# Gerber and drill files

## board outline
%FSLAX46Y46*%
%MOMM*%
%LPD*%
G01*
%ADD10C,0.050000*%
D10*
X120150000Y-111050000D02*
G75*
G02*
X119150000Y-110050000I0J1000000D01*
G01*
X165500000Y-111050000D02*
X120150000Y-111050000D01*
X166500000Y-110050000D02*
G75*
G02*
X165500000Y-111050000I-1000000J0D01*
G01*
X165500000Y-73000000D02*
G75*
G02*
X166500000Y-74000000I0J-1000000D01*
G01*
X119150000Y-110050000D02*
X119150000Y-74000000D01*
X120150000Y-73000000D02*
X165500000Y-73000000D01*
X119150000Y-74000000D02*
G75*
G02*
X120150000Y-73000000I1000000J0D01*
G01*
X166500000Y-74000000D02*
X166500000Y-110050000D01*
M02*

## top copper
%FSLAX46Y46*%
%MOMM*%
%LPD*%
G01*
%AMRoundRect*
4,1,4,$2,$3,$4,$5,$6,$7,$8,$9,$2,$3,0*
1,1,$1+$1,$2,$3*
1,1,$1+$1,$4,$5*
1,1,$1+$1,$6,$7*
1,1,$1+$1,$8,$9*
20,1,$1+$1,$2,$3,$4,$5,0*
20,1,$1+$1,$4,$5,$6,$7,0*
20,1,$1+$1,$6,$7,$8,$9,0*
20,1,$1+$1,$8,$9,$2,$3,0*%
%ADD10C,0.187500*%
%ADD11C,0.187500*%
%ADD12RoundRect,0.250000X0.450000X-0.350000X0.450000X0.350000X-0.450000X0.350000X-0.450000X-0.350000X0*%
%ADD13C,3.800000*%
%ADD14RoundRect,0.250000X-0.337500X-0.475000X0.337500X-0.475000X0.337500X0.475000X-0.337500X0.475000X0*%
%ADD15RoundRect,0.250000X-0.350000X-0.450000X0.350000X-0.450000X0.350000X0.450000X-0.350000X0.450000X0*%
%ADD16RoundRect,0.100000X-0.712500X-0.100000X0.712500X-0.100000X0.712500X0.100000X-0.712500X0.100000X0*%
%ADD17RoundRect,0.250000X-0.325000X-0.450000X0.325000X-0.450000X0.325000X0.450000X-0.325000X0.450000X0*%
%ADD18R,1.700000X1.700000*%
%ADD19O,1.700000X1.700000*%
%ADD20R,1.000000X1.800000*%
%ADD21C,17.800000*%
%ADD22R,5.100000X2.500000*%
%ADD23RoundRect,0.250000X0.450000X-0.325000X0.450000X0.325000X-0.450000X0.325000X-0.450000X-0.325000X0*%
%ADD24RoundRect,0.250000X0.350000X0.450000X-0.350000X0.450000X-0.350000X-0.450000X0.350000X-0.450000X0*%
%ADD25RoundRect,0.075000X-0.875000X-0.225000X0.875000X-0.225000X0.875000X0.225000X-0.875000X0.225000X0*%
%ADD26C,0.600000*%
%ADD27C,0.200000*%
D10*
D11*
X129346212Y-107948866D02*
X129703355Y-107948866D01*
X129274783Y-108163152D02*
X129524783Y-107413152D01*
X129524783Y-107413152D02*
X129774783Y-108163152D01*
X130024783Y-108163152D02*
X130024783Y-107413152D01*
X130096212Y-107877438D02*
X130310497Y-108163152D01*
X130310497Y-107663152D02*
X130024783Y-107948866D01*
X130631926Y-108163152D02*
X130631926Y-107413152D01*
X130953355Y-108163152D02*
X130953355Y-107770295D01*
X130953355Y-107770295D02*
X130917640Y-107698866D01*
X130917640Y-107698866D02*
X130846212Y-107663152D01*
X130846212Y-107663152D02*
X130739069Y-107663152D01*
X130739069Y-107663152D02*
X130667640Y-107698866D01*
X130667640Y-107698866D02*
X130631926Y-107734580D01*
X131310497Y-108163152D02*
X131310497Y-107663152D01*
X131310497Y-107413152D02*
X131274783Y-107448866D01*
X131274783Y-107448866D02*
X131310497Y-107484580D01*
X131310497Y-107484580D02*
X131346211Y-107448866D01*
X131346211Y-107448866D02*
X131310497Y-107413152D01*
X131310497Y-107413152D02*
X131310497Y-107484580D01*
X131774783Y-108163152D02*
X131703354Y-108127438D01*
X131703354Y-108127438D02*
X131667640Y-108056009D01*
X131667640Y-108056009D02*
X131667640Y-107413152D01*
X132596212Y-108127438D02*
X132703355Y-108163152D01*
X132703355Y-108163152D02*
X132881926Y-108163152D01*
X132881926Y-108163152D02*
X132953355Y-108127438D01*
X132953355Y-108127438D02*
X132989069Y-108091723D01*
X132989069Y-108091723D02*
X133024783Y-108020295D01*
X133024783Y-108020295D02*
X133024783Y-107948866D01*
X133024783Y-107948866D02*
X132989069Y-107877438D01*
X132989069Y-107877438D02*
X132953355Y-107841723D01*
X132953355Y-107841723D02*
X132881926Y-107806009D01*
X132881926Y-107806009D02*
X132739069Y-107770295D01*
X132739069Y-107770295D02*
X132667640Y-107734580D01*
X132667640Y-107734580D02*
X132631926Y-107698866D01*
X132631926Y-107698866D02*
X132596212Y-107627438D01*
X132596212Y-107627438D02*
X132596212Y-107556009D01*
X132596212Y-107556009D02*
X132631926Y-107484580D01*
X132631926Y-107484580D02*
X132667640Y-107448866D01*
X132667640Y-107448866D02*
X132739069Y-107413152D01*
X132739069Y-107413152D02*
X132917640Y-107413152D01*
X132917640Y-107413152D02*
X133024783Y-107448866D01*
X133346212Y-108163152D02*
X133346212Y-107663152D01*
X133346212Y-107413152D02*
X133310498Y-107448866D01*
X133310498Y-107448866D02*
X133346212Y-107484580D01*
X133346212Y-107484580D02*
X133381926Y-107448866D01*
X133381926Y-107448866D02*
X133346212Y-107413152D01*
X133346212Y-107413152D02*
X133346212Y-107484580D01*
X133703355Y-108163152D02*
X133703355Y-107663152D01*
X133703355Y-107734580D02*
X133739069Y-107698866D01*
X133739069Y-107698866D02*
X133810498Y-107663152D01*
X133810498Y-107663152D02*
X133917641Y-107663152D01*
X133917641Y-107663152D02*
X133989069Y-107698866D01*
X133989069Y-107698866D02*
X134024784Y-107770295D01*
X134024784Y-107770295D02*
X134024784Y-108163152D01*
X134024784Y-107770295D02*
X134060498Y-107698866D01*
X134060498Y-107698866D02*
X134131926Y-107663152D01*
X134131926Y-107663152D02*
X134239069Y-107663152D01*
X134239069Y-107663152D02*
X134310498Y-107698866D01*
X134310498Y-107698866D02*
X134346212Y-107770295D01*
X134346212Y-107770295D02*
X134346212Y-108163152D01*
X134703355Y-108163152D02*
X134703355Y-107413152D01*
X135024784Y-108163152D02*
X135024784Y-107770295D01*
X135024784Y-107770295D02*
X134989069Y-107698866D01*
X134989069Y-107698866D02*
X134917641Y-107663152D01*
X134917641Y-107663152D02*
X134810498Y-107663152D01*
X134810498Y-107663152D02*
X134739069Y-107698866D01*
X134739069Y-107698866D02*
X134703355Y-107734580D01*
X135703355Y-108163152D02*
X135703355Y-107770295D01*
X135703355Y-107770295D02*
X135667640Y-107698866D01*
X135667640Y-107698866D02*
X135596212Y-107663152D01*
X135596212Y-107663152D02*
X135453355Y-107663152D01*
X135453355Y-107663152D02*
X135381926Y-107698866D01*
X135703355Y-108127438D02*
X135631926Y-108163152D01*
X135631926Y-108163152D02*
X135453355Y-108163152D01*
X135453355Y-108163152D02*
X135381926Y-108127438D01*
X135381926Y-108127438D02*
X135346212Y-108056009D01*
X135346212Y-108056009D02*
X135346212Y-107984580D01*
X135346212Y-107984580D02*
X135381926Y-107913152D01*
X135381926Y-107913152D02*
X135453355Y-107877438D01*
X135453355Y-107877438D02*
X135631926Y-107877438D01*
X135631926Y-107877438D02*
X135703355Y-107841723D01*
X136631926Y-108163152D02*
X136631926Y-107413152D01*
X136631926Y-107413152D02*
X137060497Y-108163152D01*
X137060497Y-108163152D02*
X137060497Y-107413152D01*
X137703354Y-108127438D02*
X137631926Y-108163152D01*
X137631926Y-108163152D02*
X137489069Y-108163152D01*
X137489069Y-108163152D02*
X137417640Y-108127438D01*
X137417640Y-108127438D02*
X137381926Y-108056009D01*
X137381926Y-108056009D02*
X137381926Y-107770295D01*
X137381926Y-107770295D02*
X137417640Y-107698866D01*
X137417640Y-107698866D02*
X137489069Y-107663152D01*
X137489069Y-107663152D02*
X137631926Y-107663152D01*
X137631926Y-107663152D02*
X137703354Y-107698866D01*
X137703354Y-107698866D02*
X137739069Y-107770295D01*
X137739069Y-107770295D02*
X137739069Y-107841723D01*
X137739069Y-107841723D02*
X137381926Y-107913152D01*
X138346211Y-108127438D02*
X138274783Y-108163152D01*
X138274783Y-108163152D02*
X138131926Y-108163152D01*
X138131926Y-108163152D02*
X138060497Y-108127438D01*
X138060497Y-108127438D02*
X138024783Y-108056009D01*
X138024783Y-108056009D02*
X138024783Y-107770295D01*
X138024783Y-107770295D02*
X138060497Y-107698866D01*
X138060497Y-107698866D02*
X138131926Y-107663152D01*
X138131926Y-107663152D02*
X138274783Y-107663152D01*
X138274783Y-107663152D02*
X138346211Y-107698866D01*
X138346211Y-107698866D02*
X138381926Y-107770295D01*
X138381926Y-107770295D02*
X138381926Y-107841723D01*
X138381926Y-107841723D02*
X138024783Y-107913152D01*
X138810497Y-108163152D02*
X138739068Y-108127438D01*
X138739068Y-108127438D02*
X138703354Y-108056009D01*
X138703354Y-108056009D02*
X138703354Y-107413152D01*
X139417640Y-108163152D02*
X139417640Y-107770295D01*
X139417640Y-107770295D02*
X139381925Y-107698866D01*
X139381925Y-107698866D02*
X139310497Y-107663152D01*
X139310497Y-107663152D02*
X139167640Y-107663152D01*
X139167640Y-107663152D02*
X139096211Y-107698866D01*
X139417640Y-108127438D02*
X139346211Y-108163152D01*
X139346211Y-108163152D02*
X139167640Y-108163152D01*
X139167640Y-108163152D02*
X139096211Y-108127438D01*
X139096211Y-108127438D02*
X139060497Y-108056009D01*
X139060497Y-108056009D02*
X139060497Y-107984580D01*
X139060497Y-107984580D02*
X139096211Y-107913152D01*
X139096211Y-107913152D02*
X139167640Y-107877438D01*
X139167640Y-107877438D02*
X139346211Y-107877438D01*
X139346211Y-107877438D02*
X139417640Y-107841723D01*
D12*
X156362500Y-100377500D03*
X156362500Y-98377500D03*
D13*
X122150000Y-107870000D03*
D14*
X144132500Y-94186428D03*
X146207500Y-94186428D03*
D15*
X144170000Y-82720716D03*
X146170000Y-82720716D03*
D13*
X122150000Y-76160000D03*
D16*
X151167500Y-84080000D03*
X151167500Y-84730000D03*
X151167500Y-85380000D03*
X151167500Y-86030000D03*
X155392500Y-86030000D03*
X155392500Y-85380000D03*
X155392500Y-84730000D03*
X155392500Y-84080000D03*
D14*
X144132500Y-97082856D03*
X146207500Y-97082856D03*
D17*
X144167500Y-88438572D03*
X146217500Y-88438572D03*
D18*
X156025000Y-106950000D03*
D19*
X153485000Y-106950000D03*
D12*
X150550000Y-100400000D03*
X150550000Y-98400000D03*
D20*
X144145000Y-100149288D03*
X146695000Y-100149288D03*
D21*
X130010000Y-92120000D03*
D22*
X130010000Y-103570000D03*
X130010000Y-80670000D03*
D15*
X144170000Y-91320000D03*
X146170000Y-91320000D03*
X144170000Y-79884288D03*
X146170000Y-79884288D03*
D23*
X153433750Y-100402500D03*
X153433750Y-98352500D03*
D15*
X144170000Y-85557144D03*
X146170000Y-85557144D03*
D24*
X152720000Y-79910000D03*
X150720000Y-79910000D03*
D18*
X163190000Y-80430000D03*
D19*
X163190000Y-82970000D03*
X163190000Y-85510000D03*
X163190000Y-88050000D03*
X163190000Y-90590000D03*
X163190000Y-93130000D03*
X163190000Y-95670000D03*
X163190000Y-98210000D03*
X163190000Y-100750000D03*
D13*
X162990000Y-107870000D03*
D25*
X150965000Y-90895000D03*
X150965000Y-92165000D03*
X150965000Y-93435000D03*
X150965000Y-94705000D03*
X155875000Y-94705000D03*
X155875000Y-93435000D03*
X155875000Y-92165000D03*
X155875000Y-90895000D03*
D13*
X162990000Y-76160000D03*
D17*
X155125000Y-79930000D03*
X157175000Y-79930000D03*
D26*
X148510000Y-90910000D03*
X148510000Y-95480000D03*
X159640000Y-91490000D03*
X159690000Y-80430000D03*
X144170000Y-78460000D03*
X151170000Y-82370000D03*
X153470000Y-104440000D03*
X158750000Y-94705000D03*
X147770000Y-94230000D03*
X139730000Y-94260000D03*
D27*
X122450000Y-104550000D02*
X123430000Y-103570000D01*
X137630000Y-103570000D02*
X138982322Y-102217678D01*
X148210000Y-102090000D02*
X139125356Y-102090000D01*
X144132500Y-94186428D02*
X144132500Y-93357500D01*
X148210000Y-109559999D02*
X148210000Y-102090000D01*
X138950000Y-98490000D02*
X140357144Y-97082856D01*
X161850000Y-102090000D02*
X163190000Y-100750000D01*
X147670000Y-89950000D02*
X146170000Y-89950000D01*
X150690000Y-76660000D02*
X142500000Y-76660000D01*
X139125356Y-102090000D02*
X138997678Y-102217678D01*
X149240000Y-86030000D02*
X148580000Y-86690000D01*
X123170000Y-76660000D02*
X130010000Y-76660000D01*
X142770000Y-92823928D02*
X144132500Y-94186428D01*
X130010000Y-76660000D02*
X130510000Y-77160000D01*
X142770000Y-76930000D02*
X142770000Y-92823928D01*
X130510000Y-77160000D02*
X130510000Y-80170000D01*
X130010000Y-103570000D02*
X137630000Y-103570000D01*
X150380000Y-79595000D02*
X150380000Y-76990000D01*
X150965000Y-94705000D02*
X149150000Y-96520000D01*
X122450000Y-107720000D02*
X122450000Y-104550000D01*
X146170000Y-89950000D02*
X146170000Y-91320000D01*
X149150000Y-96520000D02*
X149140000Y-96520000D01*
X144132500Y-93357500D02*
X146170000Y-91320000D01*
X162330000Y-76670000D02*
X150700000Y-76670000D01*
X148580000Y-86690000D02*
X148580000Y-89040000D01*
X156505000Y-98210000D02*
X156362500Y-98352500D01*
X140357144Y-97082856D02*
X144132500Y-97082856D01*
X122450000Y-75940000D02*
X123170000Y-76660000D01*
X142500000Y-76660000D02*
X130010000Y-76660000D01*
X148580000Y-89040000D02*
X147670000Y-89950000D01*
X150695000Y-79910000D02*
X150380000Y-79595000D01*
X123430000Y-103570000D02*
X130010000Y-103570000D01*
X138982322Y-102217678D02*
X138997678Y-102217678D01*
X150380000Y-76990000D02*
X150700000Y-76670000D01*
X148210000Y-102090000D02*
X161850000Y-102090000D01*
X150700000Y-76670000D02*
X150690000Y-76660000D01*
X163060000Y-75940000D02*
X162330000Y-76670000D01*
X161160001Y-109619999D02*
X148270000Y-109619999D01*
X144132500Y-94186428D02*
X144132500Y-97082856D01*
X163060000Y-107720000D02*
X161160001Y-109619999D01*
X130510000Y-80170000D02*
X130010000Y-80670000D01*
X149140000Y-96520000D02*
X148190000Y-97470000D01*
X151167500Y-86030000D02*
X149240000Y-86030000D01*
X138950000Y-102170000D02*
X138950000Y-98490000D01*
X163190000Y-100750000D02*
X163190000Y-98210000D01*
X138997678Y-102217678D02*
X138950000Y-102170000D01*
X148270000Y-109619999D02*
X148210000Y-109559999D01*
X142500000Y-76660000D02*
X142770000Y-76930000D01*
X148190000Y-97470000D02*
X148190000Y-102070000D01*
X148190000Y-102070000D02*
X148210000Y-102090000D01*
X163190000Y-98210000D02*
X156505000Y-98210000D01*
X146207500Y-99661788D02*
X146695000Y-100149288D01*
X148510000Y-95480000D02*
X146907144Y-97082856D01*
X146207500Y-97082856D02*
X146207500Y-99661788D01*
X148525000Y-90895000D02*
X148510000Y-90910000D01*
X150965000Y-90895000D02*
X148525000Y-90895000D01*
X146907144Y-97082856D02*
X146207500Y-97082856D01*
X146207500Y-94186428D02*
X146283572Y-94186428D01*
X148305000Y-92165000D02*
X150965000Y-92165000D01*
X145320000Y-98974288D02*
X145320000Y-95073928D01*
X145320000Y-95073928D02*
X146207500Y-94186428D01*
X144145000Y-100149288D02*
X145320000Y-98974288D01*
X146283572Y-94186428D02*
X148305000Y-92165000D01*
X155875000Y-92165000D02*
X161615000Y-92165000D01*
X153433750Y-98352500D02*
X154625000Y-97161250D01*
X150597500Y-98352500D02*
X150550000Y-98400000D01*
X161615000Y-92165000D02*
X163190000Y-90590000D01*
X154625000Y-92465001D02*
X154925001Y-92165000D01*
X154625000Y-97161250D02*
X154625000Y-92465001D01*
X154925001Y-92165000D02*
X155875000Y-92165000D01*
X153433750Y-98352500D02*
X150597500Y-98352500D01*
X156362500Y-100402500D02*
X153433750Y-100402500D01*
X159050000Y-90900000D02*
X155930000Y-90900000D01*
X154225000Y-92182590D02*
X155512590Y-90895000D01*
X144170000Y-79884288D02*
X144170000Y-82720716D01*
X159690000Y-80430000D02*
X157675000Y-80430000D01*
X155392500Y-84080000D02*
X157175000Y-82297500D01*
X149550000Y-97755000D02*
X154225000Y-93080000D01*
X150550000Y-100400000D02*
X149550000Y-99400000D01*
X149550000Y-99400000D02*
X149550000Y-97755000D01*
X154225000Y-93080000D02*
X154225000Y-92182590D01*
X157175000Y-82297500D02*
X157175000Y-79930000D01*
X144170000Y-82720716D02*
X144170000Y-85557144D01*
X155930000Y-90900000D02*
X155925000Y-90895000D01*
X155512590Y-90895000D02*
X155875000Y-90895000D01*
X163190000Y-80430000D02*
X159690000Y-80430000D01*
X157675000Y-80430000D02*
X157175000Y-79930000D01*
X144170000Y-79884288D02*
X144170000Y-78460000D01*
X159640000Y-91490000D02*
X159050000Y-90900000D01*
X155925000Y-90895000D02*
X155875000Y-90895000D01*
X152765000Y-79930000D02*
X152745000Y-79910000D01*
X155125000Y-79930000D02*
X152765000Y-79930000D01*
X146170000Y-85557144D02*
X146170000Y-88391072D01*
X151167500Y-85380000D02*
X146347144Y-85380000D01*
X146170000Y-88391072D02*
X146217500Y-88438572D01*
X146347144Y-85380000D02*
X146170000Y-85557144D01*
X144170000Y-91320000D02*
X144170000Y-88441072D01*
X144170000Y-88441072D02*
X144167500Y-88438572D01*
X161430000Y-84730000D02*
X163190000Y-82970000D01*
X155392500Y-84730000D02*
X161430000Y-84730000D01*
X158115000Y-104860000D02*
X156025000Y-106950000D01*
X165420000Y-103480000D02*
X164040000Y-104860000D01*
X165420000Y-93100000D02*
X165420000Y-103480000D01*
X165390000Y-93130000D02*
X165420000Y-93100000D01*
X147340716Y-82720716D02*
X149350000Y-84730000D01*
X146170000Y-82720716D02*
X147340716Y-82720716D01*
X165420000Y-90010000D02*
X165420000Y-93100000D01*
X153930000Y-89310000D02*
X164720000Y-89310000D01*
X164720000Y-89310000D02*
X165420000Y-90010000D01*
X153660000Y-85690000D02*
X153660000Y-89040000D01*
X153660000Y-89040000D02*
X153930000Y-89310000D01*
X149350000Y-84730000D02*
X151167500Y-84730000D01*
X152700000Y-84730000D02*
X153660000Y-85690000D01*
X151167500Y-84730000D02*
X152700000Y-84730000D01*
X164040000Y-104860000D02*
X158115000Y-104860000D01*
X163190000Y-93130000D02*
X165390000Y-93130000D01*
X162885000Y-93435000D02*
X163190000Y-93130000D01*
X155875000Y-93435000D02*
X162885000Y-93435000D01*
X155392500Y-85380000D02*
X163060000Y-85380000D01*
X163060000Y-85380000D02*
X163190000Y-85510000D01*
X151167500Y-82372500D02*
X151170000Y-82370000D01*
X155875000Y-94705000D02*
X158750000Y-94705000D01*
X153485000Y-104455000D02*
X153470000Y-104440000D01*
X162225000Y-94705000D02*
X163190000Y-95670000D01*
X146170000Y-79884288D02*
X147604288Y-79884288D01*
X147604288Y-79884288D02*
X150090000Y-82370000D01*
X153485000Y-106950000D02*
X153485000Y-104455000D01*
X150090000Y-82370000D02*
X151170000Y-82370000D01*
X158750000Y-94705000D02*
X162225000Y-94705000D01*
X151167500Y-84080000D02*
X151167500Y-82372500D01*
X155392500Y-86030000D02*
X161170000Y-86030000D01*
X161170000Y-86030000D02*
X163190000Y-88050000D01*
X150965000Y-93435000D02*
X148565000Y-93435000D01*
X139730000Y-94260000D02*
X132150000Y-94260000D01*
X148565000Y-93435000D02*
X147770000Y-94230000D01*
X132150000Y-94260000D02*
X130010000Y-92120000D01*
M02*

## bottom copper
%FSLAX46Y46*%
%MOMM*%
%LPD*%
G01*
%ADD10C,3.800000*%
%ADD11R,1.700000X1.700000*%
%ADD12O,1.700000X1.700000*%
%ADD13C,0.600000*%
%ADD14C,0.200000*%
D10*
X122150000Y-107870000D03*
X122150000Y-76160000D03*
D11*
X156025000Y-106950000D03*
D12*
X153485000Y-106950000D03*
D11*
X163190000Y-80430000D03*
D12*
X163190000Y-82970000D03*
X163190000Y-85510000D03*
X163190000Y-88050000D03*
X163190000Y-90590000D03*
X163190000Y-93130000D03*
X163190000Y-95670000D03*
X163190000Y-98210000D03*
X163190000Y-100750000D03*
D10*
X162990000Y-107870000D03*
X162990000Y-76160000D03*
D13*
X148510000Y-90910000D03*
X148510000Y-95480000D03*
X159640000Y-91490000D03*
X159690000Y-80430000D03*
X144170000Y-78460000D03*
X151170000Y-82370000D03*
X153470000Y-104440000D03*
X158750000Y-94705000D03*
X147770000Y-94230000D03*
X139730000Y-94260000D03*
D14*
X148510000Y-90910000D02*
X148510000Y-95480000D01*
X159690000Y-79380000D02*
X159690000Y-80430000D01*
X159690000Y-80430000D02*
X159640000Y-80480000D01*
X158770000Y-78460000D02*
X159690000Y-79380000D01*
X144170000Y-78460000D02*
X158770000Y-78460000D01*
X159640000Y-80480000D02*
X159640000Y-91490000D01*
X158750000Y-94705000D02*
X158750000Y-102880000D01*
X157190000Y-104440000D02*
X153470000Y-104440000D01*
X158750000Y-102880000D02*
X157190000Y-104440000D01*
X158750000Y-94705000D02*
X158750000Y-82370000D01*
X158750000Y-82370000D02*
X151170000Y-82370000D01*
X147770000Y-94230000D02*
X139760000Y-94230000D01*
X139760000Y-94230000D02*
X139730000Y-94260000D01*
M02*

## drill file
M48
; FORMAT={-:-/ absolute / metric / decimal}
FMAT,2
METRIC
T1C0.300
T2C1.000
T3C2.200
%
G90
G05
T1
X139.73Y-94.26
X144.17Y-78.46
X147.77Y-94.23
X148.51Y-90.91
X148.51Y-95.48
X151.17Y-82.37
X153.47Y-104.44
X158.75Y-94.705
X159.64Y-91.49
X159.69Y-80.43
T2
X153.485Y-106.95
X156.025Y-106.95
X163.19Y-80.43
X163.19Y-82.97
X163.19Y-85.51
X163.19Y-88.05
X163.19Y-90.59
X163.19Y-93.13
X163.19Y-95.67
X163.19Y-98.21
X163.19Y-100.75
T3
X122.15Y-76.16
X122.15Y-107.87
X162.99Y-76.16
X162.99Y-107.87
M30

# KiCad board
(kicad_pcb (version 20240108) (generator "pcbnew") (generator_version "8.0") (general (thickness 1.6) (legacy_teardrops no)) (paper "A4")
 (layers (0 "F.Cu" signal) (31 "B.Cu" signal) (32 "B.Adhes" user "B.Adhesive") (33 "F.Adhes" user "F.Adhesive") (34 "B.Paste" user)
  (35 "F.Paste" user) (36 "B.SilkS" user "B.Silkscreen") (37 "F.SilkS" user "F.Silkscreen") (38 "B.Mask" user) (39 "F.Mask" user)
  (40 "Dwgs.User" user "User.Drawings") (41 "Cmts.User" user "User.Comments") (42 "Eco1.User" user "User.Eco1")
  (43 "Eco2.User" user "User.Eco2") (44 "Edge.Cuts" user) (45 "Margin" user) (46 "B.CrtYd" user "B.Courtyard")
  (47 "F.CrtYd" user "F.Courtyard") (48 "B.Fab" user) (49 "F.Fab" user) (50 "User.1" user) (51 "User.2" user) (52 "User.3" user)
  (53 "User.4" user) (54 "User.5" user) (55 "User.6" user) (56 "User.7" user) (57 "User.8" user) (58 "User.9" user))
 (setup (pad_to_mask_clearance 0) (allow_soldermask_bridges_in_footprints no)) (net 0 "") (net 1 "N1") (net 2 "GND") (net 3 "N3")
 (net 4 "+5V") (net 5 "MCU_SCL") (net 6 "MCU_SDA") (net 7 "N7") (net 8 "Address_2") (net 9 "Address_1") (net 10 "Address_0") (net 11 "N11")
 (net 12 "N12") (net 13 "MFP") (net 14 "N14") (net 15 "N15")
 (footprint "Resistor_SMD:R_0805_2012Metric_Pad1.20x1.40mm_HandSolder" (layer "F.Cu") (at 156.3625 99.3775 90)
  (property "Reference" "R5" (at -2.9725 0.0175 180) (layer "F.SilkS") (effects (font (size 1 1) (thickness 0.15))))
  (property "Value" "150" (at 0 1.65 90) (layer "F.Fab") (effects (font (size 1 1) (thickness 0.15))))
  (pad "1" smd roundrect (at -1 0 90) (size 1.2 1.4) (layers "F.Cu" "F.Paste" "F.Mask") (roundrect_rratio 0.208333) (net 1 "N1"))
  (pad "2" smd roundrect (at 1 0 90) (size 1.2 1.4) (layers "F.Cu" "F.Paste" "F.Mask") (roundrect_rratio 0.208333) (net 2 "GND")))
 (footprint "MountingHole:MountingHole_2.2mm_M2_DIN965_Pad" (layer "F.Cu") (at 122.15 107.87)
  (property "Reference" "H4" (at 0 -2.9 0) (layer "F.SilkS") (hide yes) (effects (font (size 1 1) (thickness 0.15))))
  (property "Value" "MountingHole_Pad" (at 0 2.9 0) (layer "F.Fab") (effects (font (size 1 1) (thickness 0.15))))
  (pad "1" thru_hole circle (at 0 0) (size 3.8 3.8) (drill 2.2) (layers "*.Cu" "*.Mask") (remove_unused_layers no) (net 2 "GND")))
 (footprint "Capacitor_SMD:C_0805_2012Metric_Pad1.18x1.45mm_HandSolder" (layer "F.Cu") (at 145.17 94.186428)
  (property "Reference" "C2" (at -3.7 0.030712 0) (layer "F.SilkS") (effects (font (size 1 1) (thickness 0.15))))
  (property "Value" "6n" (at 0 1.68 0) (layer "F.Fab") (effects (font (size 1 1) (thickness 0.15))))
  (pad "1" smd roundrect (at -1.0375 0) (size 1.175 1.45) (layers "F.Cu" "F.Paste" "F.Mask") (roundrect_rratio 0.212766) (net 2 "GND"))
  (pad "2" smd roundrect (at 1.0375 0) (size 1.175 1.45) (layers "F.Cu" "F.Paste" "F.Mask") (roundrect_rratio 0.212766) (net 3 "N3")))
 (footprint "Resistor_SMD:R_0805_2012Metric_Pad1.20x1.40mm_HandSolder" (layer "F.Cu") (at 145.17 82.720716)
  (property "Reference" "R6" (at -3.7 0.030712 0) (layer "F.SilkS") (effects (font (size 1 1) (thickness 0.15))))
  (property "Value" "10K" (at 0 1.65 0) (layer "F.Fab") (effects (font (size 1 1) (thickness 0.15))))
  (pad "1" smd roundrect (at -1 0) (size 1.2 1.4) (layers "F.Cu" "F.Paste" "F.Mask") (roundrect_rratio 0.208333) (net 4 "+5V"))
  (pad "2" smd roundrect (at 1 0) (size 1.2 1.4) (layers "F.Cu" "F.Paste" "F.Mask") (roundrect_rratio 0.208333) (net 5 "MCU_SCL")))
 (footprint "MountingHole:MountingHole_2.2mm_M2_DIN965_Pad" (layer "F.Cu") (at 122.15 76.16)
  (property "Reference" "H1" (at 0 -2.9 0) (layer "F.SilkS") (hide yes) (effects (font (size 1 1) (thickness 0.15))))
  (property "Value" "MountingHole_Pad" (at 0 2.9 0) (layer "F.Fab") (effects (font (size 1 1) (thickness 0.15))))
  (pad "1" thru_hole circle (at 0 0) (size 3.8 3.8) (drill 2.2) (layers "*.Cu" "*.Mask") (remove_unused_layers no) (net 2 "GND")))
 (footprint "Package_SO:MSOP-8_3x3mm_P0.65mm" (layer "F.Cu") (at 153.28 85.055)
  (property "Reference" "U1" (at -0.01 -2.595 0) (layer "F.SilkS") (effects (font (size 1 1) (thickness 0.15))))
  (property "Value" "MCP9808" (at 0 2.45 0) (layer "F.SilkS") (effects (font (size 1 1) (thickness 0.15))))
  (pad "1" smd roundrect (at -2.1125 -0.975) (size 1.625 0.4) (layers "F.Cu" "F.Paste" "F.Mask") (roundrect_rratio 0.25) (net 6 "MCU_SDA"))
  (pad "2" smd roundrect (at -2.1125 -0.325) (size 1.625 0.4) (layers "F.Cu" "F.Paste" "F.Mask") (roundrect_rratio 0.25) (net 5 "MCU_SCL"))
  (pad "3" smd roundrect (at -2.1125 0.325) (size 1.625 0.4) (layers "F.Cu" "F.Paste" "F.Mask") (roundrect_rratio 0.25) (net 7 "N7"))
  (pad "4" smd roundrect (at -2.1125 0.975) (size 1.625 0.4) (layers "F.Cu" "F.Paste" "F.Mask") (roundrect_rratio 0.25) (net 2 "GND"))
  (pad "5" smd roundrect (at 2.1125 0.975) (size 1.625 0.4) (layers "F.Cu" "F.Paste" "F.Mask") (roundrect_rratio 0.25) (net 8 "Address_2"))
  (pad "6" smd roundrect (at 2.1125 0.325) (size 1.625 0.4) (layers "F.Cu" "F.Paste" "F.Mask") (roundrect_rratio 0.25) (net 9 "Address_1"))
  (pad "7" smd roundrect (at 2.1125 -0.325) (size 1.625 0.4) (layers "F.Cu" "F.Paste" "F.Mask") (roundrect_rratio 0.25) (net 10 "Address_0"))
  (pad "8" smd roundrect (at 2.1125 -0.975) (size 1.625 0.4) (layers "F.Cu" "F.Paste" "F.Mask") (roundrect_rratio 0.25) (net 4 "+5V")))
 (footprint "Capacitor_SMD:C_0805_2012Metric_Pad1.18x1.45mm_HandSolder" (layer "F.Cu") (at 145.17 97.082856)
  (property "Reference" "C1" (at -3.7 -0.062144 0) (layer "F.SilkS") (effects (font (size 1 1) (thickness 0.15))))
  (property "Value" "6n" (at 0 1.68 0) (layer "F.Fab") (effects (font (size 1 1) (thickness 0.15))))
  (pad "1" smd roundrect (at -1.0375 0) (size 1.175 1.45) (layers "F.Cu" "F.Paste" "F.Mask") (roundrect_rratio 0.212766) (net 2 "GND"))
  (pad "2" smd roundrect (at 1.0375 0) (size 1.175 1.45) (layers "F.Cu" "F.Paste" "F.Mask") (roundrect_rratio 0.212766) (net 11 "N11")))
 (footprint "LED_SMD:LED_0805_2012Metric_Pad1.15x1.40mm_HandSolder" (layer "F.Cu") (at 145.1925 88.438572)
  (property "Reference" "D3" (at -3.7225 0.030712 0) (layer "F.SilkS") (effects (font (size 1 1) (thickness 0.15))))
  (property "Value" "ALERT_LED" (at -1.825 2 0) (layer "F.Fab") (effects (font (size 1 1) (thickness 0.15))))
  (pad "1" smd roundrect (at -1.025 0) (size 1.15 1.4) (layers "F.Cu" "F.Paste" "F.Mask") (roundrect_rratio 0.217391) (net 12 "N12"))
  (pad "2" smd roundrect (at 1.025 0) (size 1.15 1.4) (layers "F.Cu" "F.Paste" "F.Mask") (roundrect_rratio 0.217391) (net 7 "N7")))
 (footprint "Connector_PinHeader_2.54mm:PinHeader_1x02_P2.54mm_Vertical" (layer "F.Cu") (at 156.025 106.95 -90)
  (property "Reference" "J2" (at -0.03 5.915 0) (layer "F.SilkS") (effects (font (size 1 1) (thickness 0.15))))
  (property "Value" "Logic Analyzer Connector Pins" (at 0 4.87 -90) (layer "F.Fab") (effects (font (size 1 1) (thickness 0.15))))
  (pad "1" thru_hole rect (at 0 0 270) (size 1.7 1.7) (drill 1) (layers "*.Cu" "*.Mask") (remove_unused_layers no) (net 5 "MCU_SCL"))
  (pad "2" thru_hole oval (at 0 2.54 270) (size 1.7 1.7) (drill 1) (layers "*.Cu" "*.Mask") (remove_unused_layers no) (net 6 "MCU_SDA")))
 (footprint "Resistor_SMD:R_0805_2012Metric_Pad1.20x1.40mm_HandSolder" (layer "F.Cu") (at 150.55 99.4 90)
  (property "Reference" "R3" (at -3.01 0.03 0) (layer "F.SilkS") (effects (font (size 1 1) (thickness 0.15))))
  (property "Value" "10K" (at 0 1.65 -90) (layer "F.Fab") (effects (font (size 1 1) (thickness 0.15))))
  (pad "1" smd roundrect (at -1 0 90) (size 1.2 1.4) (layers "F.Cu" "F.Paste" "F.Mask") (roundrect_rratio 0.208333) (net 4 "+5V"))
  (pad "2" smd roundrect (at 1 0 90) (size 1.2 1.4) (layers "F.Cu" "F.Paste" "F.Mask") (roundrect_rratio 0.208333) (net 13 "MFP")))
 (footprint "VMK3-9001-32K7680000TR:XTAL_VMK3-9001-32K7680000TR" (layer "F.Cu") (at 145.42 100.149288)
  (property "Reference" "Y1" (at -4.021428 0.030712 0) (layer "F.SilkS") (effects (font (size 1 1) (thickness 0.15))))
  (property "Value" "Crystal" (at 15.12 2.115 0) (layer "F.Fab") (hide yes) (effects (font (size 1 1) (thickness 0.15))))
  (pad "1" smd rect (at -1.275 0) (size 1 1.8) (layers "F.Cu" "F.Paste" "F.Mask") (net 3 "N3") (solder_mask_margin 0.102))
  (pad "2" smd rect (at 1.275 0) (size 1 1.8) (layers "F.Cu" "F.Paste" "F.Mask") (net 11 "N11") (solder_mask_margin 0.102)))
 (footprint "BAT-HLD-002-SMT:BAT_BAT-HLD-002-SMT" (layer "F.Cu") (at 130.01 92.12 90)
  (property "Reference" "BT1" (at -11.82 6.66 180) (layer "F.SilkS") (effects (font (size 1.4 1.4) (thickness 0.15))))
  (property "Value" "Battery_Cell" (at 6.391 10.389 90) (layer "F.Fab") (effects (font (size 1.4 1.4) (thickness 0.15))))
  (pad "N" smd circle (at 0 0 90) (size 17.8 17.8) (layers "F.Cu" "F.Mask") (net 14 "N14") (solder_mask_margin 0.102))
  (pad "P1" smd rect (at -11.45 0 90) (size 2.5 5.1) (layers "F.Cu" "F.Paste" "F.Mask") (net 2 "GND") (solder_mask_margin 0.102))
  (pad "P2" smd rect (at 11.45 0 90) (size 2.5 5.1) (layers "F.Cu" "F.Paste" "F.Mask") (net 2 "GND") (solder_mask_margin 0.102)))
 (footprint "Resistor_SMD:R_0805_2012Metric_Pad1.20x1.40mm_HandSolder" (layer "F.Cu") (at 145.17 91.32)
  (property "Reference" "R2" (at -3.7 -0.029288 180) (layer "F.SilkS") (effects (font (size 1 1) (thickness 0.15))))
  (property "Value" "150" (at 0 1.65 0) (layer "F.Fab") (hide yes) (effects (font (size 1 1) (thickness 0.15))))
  (pad "1" smd roundrect (at -1 0) (size 1.2 1.4) (layers "F.Cu" "F.Paste" "F.Mask") (roundrect_rratio 0.208333) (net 12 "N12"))
  (pad "2" smd roundrect (at 1 0) (size 1.2 1.4) (layers "F.Cu" "F.Paste" "F.Mask") (roundrect_rratio 0.208333) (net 2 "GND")))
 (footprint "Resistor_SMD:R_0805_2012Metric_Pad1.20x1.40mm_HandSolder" (layer "F.Cu") (at 145.17 79.884288)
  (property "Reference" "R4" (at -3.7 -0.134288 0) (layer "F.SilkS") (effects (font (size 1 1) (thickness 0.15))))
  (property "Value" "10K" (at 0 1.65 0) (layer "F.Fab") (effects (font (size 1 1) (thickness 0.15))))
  (pad "1" smd roundrect (at -1 0) (size 1.2 1.4) (layers "F.Cu" "F.Paste" "F.Mask") (roundrect_rratio 0.208333) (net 4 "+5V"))
  (pad "2" smd roundrect (at 1 0) (size 1.2 1.4) (layers "F.Cu" "F.Paste" "F.Mask") (roundrect_rratio 0.208333) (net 6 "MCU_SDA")))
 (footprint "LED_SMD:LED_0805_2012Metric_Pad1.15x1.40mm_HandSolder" (layer "F.Cu") (at 153.43375 99.3775 90)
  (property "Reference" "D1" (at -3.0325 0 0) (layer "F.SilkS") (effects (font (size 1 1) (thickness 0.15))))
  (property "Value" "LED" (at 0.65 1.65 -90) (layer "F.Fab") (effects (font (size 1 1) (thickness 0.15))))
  (pad "1" smd roundrect (at -1.025 0 90) (size 1.15 1.4) (layers "F.Cu" "F.Paste" "F.Mask") (roundrect_rratio 0.217391) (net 1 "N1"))
  (pad "2" smd roundrect (at 1.025 0 90) (size 1.15 1.4) (layers "F.Cu" "F.Paste" "F.Mask") (roundrect_rratio 0.217391) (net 13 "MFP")))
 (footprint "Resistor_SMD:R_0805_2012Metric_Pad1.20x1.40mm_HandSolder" (layer "F.Cu") (at 145.17 85.557144)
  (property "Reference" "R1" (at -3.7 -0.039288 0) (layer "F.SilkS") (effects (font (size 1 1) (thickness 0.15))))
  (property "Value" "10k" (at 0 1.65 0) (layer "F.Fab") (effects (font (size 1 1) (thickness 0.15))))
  (pad "1" smd roundrect (at -1 0) (size 1.2 1.4) (layers "F.Cu" "F.Paste" "F.Mask") (roundrect_rratio 0.208333) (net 4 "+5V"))
  (pad "2" smd roundrect (at 1 0) (size 1.2 1.4) (layers "F.Cu" "F.Paste" "F.Mask") (roundrect_rratio 0.208333) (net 7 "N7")))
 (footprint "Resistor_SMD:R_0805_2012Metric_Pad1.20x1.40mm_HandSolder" (layer "F.Cu") (at 151.72 79.91 180)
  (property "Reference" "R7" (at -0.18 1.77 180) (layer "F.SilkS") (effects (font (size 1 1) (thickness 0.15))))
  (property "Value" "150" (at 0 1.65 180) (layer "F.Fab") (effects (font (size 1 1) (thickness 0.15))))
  (pad "1" smd roundrect (at -1 0 180) (size 1.2 1.4) (layers "F.Cu" "F.Paste" "F.Mask") (roundrect_rratio 0.208333) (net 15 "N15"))
  (pad "2" smd roundrect (at 1 0 180) (size 1.2 1.4) (layers "F.Cu" "F.Paste" "F.Mask") (roundrect_rratio 0.208333) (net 2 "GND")))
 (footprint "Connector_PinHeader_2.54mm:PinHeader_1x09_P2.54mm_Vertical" (layer "F.Cu") (at 163.19 80.43)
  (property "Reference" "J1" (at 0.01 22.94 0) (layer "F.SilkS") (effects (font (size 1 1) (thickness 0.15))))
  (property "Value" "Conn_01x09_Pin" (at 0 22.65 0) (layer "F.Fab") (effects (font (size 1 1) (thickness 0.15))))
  (pad "1" thru_hole rect (at 0 0) (size 1.7 1.7) (drill 1) (layers "*.Cu" "*.Mask") (remove_unused_layers no) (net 4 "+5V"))
  (pad "2" thru_hole oval (at 0 2.54) (size 1.7 1.7) (drill 1) (layers "*.Cu" "*.Mask") (remove_unused_layers no) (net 10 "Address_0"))
  (pad "3" thru_hole oval (at 0 5.08) (size 1.7 1.7) (drill 1) (layers "*.Cu" "*.Mask") (remove_unused_layers no) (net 9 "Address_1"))
  (pad "4" thru_hole oval (at 0 7.62) (size 1.7 1.7) (drill 1) (layers "*.Cu" "*.Mask") (remove_unused_layers no) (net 8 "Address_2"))
  (pad "5" thru_hole oval (at 0 10.16) (size 1.7 1.7) (drill 1) (layers "*.Cu" "*.Mask") (remove_unused_layers no) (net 13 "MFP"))
  (pad "6" thru_hole oval (at 0 12.7) (size 1.7 1.7) (drill 1) (layers "*.Cu" "*.Mask") (remove_unused_layers no) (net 5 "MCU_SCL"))
  (pad "7" thru_hole oval (at 0 15.24) (size 1.7 1.7) (drill 1) (layers "*.Cu" "*.Mask") (remove_unused_layers no) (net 6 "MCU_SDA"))
  (pad "8" thru_hole oval (at 0 17.78) (size 1.7 1.7) (drill 1) (layers "*.Cu" "*.Mask") (remove_unused_layers no) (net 2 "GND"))
  (pad "9" thru_hole oval (at 0 20.32) (size 1.7 1.7) (drill 1) (layers "*.Cu" "*.Mask") (remove_unused_layers no) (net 2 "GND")))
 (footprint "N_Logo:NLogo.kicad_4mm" (layer "F.Cu") (at 127.06 107.719644)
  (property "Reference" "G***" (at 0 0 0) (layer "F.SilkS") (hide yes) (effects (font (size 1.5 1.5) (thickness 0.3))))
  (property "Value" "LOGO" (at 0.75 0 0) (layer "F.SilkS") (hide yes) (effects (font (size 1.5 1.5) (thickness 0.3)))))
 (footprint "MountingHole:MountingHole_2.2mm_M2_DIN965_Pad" (layer "F.Cu") (at 162.99 107.87)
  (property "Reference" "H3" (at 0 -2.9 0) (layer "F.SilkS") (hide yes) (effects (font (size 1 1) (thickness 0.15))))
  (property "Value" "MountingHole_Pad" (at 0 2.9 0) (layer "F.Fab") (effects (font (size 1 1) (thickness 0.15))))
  (pad "1" thru_hole circle (at 0 0) (size 3.8 3.8) (drill 2.2) (layers "*.Cu" "*.Mask") (remove_unused_layers no) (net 2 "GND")))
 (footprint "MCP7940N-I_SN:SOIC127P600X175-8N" (layer "F.Cu") (at 153.42 92.8)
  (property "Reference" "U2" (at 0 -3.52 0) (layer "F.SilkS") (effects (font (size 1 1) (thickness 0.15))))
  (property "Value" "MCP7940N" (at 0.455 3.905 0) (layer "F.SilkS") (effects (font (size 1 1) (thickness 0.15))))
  (pad "1" smd roundrect (at -2.455 -1.905) (size 1.9 0.6) (layers "F.Cu" "F.Paste" "F.Mask") (roundrect_rratio 0.125) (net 11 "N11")
   (solder_mask_margin 0.102))
  (pad "2" smd roundrect (at -2.455 -0.635) (size 1.9 0.6) (layers "F.Cu" "F.Paste" "F.Mask") (roundrect_rratio 0.125) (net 3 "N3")
   (solder_mask_margin 0.102))
  (pad "3" smd roundrect (at -2.455 0.635) (size 1.9 0.6) (layers "F.Cu" "F.Paste" "F.Mask") (roundrect_rratio 0.125) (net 14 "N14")
   (solder_mask_margin 0.102))
  (pad "4" smd roundrect (at -2.455 1.905) (size 1.9 0.6) (layers "F.Cu" "F.Paste" "F.Mask") (roundrect_rratio 0.125) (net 2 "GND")
   (solder_mask_margin 0.102))
  (pad "5" smd roundrect (at 2.455 1.905) (size 1.9 0.6) (layers "F.Cu" "F.Paste" "F.Mask") (roundrect_rratio 0.125) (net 6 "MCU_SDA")
   (solder_mask_margin 0.102))
  (pad "6" smd roundrect (at 2.455 0.635) (size 1.9 0.6) (layers "F.Cu" "F.Paste" "F.Mask") (roundrect_rratio 0.125) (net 5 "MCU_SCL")
   (solder_mask_margin 0.102))
  (pad "7" smd roundrect (at 2.455 -0.635) (size 1.9 0.6) (layers "F.Cu" "F.Paste" "F.Mask") (roundrect_rratio 0.125) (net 13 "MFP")
   (solder_mask_margin 0.102))
  (pad "8" smd roundrect (at 2.455 -1.905) (size 1.9 0.6) (layers "F.Cu" "F.Paste" "F.Mask") (roundrect_rratio 0.125) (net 4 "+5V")
   (solder_mask_margin 0.102)))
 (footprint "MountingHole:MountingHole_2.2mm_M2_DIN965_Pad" (layer "F.Cu") (at 162.99 76.16)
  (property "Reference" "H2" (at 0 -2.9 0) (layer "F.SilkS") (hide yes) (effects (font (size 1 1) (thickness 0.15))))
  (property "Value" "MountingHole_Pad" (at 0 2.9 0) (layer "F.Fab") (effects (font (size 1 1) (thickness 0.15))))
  (pad "1" thru_hole circle (at 0 0) (size 3.8 3.8) (drill 2.2) (layers "*.Cu" "*.Mask") (remove_unused_layers no) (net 2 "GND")))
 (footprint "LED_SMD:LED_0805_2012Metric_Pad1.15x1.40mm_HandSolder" (layer "F.Cu") (at 156.15 79.93)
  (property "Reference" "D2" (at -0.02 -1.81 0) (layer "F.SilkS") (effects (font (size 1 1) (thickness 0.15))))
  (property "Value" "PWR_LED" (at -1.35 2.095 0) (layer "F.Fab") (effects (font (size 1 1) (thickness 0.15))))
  (pad "1" smd roundrect (at -1.025 0) (size 1.15 1.4) (layers "F.Cu" "F.Paste" "F.Mask") (roundrect_rratio 0.217391) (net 15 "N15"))
  (pad "2" smd roundrect (at 1.025 0) (size 1.15 1.4) (layers "F.Cu" "F.Paste" "F.Mask") (roundrect_rratio 0.217391) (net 4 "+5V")))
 (gr_arc (start 120.15 111.05) (mid 119.442893 110.757107) (end 119.15 110.05) (stroke (width 0.05) (type default)) (layer "Edge.Cuts"))
 (gr_line (start 165.5 111.05) (end 120.15 111.05) (stroke (width 0.05) (type default)) (layer "Edge.Cuts"))
 (gr_arc (start 166.5 110.05) (mid 166.207107 110.757107) (end 165.5 111.05) (stroke (width 0.05) (type default)) (layer "Edge.Cuts"))
 (gr_arc (start 165.5 73) (mid 166.207107 73.292893) (end 166.5 74) (stroke (width 0.05) (type default)) (layer "Edge.Cuts"))
 (gr_line (start 119.15 110.05) (end 119.15 74) (stroke (width 0.05) (type default)) (layer "Edge.Cuts"))
 (gr_line (start 120.15 73) (end 165.5 73) (stroke (width 0.05) (type default)) (layer "Edge.Cuts"))
 (gr_arc (start 119.15 74) (mid 119.442893 73.292893) (end 120.15 73) (stroke (width 0.05) (type default)) (layer "Edge.Cuts"))
 (gr_line (start 166.5 74) (end 166.5 110.05) (stroke (width 0.05) (type default)) (layer "Edge.Cuts"))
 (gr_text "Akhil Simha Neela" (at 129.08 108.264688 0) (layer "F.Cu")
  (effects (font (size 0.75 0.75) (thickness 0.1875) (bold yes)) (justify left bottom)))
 (segment (start 122.45 104.55) (end 123.43 103.57) (width 0.2) (layer "F.Cu") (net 2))
 (segment (start 137.63 103.57) (end 138.982322 102.217678) (width 0.2) (layer "F.Cu") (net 2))
 (segment (start 148.21 102.09) (end 139.125356 102.09) (width 0.2) (layer "F.Cu") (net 2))
 (segment (start 144.1325 94.186428) (end 144.1325 93.3575) (width 0.2) (layer "F.Cu") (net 2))
 (segment (start 148.21 109.559999) (end 148.21 102.09) (width 0.2) (layer "F.Cu") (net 2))
 (segment (start 138.95 98.49) (end 140.357144 97.082856) (width 0.2) (layer "F.Cu") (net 2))
 (segment (start 161.85 102.09) (end 163.19 100.75) (width 0.2) (layer "F.Cu") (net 2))
 (segment (start 147.67 89.95) (end 146.17 89.95) (width 0.2) (layer "F.Cu") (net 2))
 (segment (start 150.69 76.66) (end 142.5 76.66) (width 0.2) (layer "F.Cu") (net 2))
 (segment (start 139.125356 102.09) (end 138.997678 102.217678) (width 0.2) (layer "F.Cu") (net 2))
 (segment (start 149.24 86.03) (end 148.58 86.69) (width 0.2) (layer "F.Cu") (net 2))
 (segment (start 123.17 76.66) (end 130.01 76.66) (width 0.2) (layer "F.Cu") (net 2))
 (segment (start 142.77 92.823928) (end 144.1325 94.186428) (width 0.2) (layer "F.Cu") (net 2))
 (segment (start 130.01 76.66) (end 130.51 77.16) (width 0.2) (layer "F.Cu") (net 2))
 (segment (start 142.77 76.93) (end 142.77 92.823928) (width 0.2) (layer "F.Cu") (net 2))
 (segment (start 130.51 77.16) (end 130.51 80.17) (width 0.2) (layer "F.Cu") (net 2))
 (segment (start 130.01 103.57) (end 137.63 103.57) (width 0.2) (layer "F.Cu") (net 2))
 (segment (start 150.38 79.595) (end 150.38 76.99) (width 0.2) (layer "F.Cu") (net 2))
 (segment (start 150.965 94.705) (end 149.15 96.52) (width 0.2) (layer "F.Cu") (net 2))
 (segment (start 122.45 107.72) (end 122.45 104.55) (width 0.2) (layer "F.Cu") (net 2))
 (segment (start 146.17 89.95) (end 146.17 91.32) (width 0.2) (layer "F.Cu") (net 2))
 (segment (start 149.15 96.52) (end 149.14 96.52) (width 0.2) (layer "F.Cu") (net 2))
 (segment (start 144.1325 93.3575) (end 146.17 91.32) (width 0.2) (layer "F.Cu") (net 2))
 (segment (start 162.33 76.67) (end 150.7 76.67) (width 0.2) (layer "F.Cu") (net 2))
 (segment (start 148.58 86.69) (end 148.58 89.04) (width 0.2) (layer "F.Cu") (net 2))
 (segment (start 156.505 98.21) (end 156.3625 98.3525) (width 0.2) (layer "F.Cu") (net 2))
 (segment (start 140.357144 97.082856) (end 144.1325 97.082856) (width 0.2) (layer "F.Cu") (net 2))
 (segment (start 122.45 75.94) (end 123.17 76.66) (width 0.2) (layer "F.Cu") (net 2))
 (segment (start 142.5 76.66) (end 130.01 76.66) (width 0.2) (layer "F.Cu") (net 2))
 (segment (start 148.58 89.04) (end 147.67 89.95) (width 0.2) (layer "F.Cu") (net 2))
 (segment (start 150.695 79.91) (end 150.38 79.595) (width 0.2) (layer "F.Cu") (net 2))
 (segment (start 123.43 103.57) (end 130.01 103.57) (width 0.2) (layer "F.Cu") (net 2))
 (segment (start 138.982322 102.217678) (end 138.997678 102.217678) (width 0.2) (layer "F.Cu") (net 2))
 (segment (start 150.38 76.99) (end 150.7 76.67) (width 0.2) (layer "F.Cu") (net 2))
 (segment (start 148.21 102.09) (end 161.85 102.09) (width 0.2) (layer "F.Cu") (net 2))
 (segment (start 150.7 76.67) (end 150.69 76.66) (width 0.2) (layer "F.Cu") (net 2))
 (segment (start 163.06 75.94) (end 162.33 76.67) (width 0.2) (layer "F.Cu") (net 2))
 (segment (start 161.160001 109.619999) (end 148.27 109.619999) (width 0.2) (layer "F.Cu") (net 2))
 (segment (start 144.1325 94.186428) (end 144.1325 97.082856) (width 0.2) (layer "F.Cu") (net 2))
 (segment (start 163.06 107.72) (end 161.160001 109.619999) (width 0.2) (layer "F.Cu") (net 2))
 (segment (start 130.51 80.17) (end 130.01 80.67) (width 0.2) (layer "F.Cu") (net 2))
 (segment (start 149.14 96.52) (end 148.19 97.47) (width 0.2) (layer "F.Cu") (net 2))
 (segment (start 151.1675 86.03) (end 149.24 86.03) (width 0.2) (layer "F.Cu") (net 2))
 (segment (start 138.95 102.17) (end 138.95 98.49) (width 0.2) (layer "F.Cu") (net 2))
 (segment (start 163.19 100.75) (end 163.19 98.21) (width 0.2) (layer "F.Cu") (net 2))
 (segment (start 138.997678 102.217678) (end 138.95 102.17) (width 0.2) (layer "F.Cu") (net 2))
 (segment (start 148.27 109.619999) (end 148.21 109.559999) (width 0.2) (layer "F.Cu") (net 2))
 (segment (start 142.5 76.66) (end 142.77 76.93) (width 0.2) (layer "F.Cu") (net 2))
 (segment (start 148.19 97.47) (end 148.19 102.07) (width 0.2) (layer "F.Cu") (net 2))
 (segment (start 148.19 102.07) (end 148.21 102.09) (width 0.2) (layer "F.Cu") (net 2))
 (segment (start 163.19 98.21) (end 156.505 98.21) (width 0.2) (layer "F.Cu") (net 2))
 (segment (start 146.2075 99.661788) (end 146.695 100.149288) (width 0.2) (layer "F.Cu") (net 11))
 (segment (start 148.51 95.48) (end 146.907144 97.082856) (width 0.2) (layer "F.Cu") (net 11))
 (segment (start 146.2075 97.082856) (end 146.2075 99.661788) (width 0.2) (layer "F.Cu") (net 11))
 (segment (start 148.525 90.895) (end 148.51 90.91) (width 0.2) (layer "F.Cu") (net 11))
 (segment (start 150.965 90.895) (end 148.525 90.895) (width 0.2) (layer "F.Cu") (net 11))
 (segment (start 146.907144 97.082856) (end 146.2075 97.082856) (width 0.2) (layer "F.Cu") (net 11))
 (via (at 148.51 90.91) (size 0.6) (drill 0.3) (layers "F.Cu" "B.Cu") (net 11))
 (via (at 148.51 95.48) (size 0.6) (drill 0.3) (layers "F.Cu" "B.Cu") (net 11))
 (segment (start 148.51 90.91) (end 148.51 95.48) (width 0.2) (layer "B.Cu") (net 11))
 (segment (start 146.2075 94.186428) (end 146.283572 94.186428) (width 0.2) (layer "F.Cu") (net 3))
 (segment (start 148.305 92.165) (end 150.965 92.165) (width 0.2) (layer "F.Cu") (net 3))
 (segment (start 145.32 98.974288) (end 145.32 95.073928) (width 0.2) (layer "F.Cu") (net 3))
 (segment (start 145.32 95.073928) (end 146.2075 94.186428) (width 0.2) (layer "F.Cu") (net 3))
 (segment (start 144.145 100.149288) (end 145.32 98.974288) (width 0.2) (layer "F.Cu") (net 3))
 (segment (start 146.283572 94.186428) (end 148.305 92.165) (width 0.2) (layer "F.Cu") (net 3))
 (segment (start 155.875 92.165) (end 161.615 92.165) (width 0.2) (layer "F.Cu") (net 13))
 (segment (start 153.43375 98.3525) (end 154.625 97.16125) (width 0.2) (layer "F.Cu") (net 13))
 (segment (start 150.5975 98.3525) (end 150.55 98.4) (width 0.2) (layer "F.Cu") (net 13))
 (segment (start 161.615 92.165) (end 163.19 90.59) (width 0.2) (layer "F.Cu") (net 13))
 (segment (start 154.625 92.465001) (end 154.925001 92.165) (width 0.2) (layer "F.Cu") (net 13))
 (segment (start 154.625 97.16125) (end 154.625 92.465001) (width 0.2) (layer "F.Cu") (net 13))
 (segment (start 154.925001 92.165) (end 155.875 92.165) (width 0.2) (layer "F.Cu") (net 13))
 (segment (start 153.43375 98.3525) (end 150.5975 98.3525) (width 0.2) (layer "F.Cu") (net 13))
 (segment (start 156.3625 100.4025) (end 153.43375 100.4025) (width 0.2) (layer "F.Cu") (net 1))
 (segment (start 159.05 90.9) (end 155.93 90.9) (width 0.2) (layer "F.Cu") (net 4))
 (segment (start 154.225 92.18259) (end 155.51259 90.895) (width 0.2) (layer "F.Cu") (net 4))
 (segment (start 144.17 79.884288) (end 144.17 82.720716) (width 0.2) (layer "F.Cu") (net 4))
 (segment (start 159.69 80.43) (end 157.675 80.43) (width 0.2) (layer "F.Cu") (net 4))
 (segment (start 155.3925 84.08) (end 157.175 82.2975) (width 0.2) (layer "F.Cu") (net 4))
 (segment (start 149.55 97.755) (end 154.225 93.08) (width 0.2) (layer "F.Cu") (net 4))
 (segment (start 150.55 100.4) (end 149.55 99.4) (width 0.2) (layer "F.Cu") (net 4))
 (segment (start 149.55 99.4) (end 149.55 97.755) (width 0.2) (layer "F.Cu") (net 4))
 (segment (start 154.225 93.08) (end 154.225 92.18259) (width 0.2) (layer "F.Cu") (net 4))
 (segment (start 157.175 82.2975) (end 157.175 79.93) (width 0.2) (layer "F.Cu") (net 4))
 (segment (start 144.17 82.720716) (end 144.17 85.557144) (width 0.2) (layer "F.Cu") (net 4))
 (segment (start 155.93 90.9) (end 155.925 90.895) (width 0.2) (layer "F.Cu") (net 4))
 (segment (start 155.51259 90.895) (end 155.875 90.895) (width 0.2) (layer "F.Cu") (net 4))
 (segment (start 163.19 80.43) (end 159.69 80.43) (width 0.2) (layer "F.Cu") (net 4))
 (segment (start 157.675 80.43) (end 157.175 79.93) (width 0.2) (layer "F.Cu") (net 4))
 (segment (start 144.17 79.884288) (end 144.17 78.46) (width 0.2) (layer "F.Cu") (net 4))
 (segment (start 159.64 91.49) (end 159.05 90.9) (width 0.2) (layer "F.Cu") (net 4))
 (segment (start 155.925 90.895) (end 155.875 90.895) (width 0.2) (layer "F.Cu") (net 4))
 (via (at 159.64 91.49) (size 0.6) (drill 0.3) (layers "F.Cu" "B.Cu") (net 4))
 (via (at 159.69 80.43) (size 0.6) (drill 0.3) (layers "F.Cu" "B.Cu") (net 4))
 (via (at 144.17 78.46) (size 0.6) (drill 0.3) (layers "F.Cu" "B.Cu") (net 4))
 (segment (start 159.69 79.38) (end 159.69 80.43) (width 0.2) (layer "B.Cu") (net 4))
 (segment (start 159.69 80.43) (end 159.64 80.48) (width 0.2) (layer "B.Cu") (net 4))
 (segment (start 158.77 78.46) (end 159.69 79.38) (width 0.2) (layer "B.Cu") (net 4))
 (segment (start 144.17 78.46) (end 158.77 78.46) (width 0.2) (layer "B.Cu") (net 4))
 (segment (start 159.64 80.48) (end 159.64 91.49) (width 0.2) (layer "B.Cu") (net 4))
 (segment (start 152.765 79.93) (end 152.745 79.91) (width 0.2) (layer "F.Cu") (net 15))
 (segment (start 155.125 79.93) (end 152.765 79.93) (width 0.2) (layer "F.Cu") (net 15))
 (segment (start 146.17 85.557144) (end 146.17 88.391072) (width 0.2) (layer "F.Cu") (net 7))
 (segment (start 151.1675 85.38) (end 146.347144 85.38) (width 0.2) (layer "F.Cu") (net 7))
 (segment (start 146.17 88.391072) (end 146.2175 88.438572) (width 0.2) (layer "F.Cu") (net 7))
 (segment (start 146.347144 85.38) (end 146.17 85.557144) (width 0.2) (layer "F.Cu") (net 7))
 (segment (start 144.17 91.32) (end 144.17 88.441072) (width 0.2) (layer "F.Cu") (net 12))
 (segment (start 144.17 88.441072) (end 144.1675 88.438572) (width 0.2) (layer "F.Cu") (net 12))
 (segment (start 161.43 84.73) (end 163.19 82.97) (width 0.2) (layer "F.Cu") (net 10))
 (segment (start 155.3925 84.73) (end 161.43 84.73) (width 0.2) (layer "F.Cu") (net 10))
 (segment (start 158.115 104.86) (end 156.025 106.95) (width 0.2) (layer "F.Cu") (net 5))
 (segment (start 165.42 103.48) (end 164.04 104.86) (width 0.2) (layer "F.Cu") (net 5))
 (segment (start 165.42 93.1) (end 165.42 103.48) (width 0.2) (layer "F.Cu") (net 5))
 (segment (start 165.39 93.13) (end 165.42 93.1) (width 0.2) (layer "F.Cu") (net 5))
 (segment (start 147.340716 82.720716) (end 149.35 84.73) (width 0.2) (layer "F.Cu") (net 5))
 (segment (start 146.17 82.720716) (end 147.340716 82.720716) (width 0.2) (layer "F.Cu") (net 5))
 (segment (start 165.42 90.01) (end 165.42 93.1) (width 0.2) (layer "F.Cu") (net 5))
 (segment (start 153.93 89.31) (end 164.72 89.31) (width 0.2) (layer "F.Cu") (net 5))
 (segment (start 164.72 89.31) (end 165.42 90.01) (width 0.2) (layer "F.Cu") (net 5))
 (segment (start 153.66 85.69) (end 153.66 89.04) (width 0.2) (layer "F.Cu") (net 5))
 (segment (start 153.66 89.04) (end 153.93 89.31) (width 0.2) (layer "F.Cu") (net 5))
 (segment (start 149.35 84.73) (end 151.1675 84.73) (width 0.2) (layer "F.Cu") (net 5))
 (segment (start 152.7 84.73) (end 153.66 85.69) (width 0.2) (layer "F.Cu") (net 5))
 (segment (start 151.1675 84.73) (end 152.7 84.73) (width 0.2) (layer "F.Cu") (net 5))
 (segment (start 164.04 104.86) (end 158.115 104.86) (width 0.2) (layer "F.Cu") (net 5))
 (segment (start 163.19 93.13) (end 165.39 93.13) (width 0.2) (layer "F.Cu") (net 5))
 (segment (start 162.885 93.435) (end 163.19 93.13) (width 0.2) (layer "F.Cu") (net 5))
 (segment (start 155.875 93.435) (end 162.885 93.435) (width 0.2) (layer "F.Cu") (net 5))
 (segment (start 155.3925 85.38) (end 163.06 85.38) (width 0.2) (layer "F.Cu") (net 9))
 (segment (start 163.06 85.38) (end 163.19 85.51) (width 0.2) (layer "F.Cu") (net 9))
 (segment (start 151.1675 82.3725) (end 151.17 82.37) (width 0.2) (layer "F.Cu") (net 6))
 (segment (start 155.875 94.705) (end 158.75 94.705) (width 0.2) (layer "F.Cu") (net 6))
 (segment (start 153.485 104.455) (end 153.47 104.44) (width 0.2) (layer "F.Cu") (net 6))
 (segment (start 162.225 94.705) (end 163.19 95.67) (width 0.2) (layer "F.Cu") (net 6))
 (segment (start 146.17 79.884288) (end 147.604288 79.884288) (width 0.2) (layer "F.Cu") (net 6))
 (segment (start 147.604288 79.884288) (end 150.09 82.37) (width 0.2) (layer "F.Cu") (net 6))
 (segment (start 153.485 106.95) (end 153.485 104.455) (width 0.2) (layer "F.Cu") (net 6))
 (segment (start 150.09 82.37) (end 151.17 82.37) (width 0.2) (layer "F.Cu") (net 6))
 (segment (start 158.75 94.705) (end 162.225 94.705) (width 0.2) (layer "F.Cu") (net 6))
 (segment (start 151.1675 84.08) (end 151.1675 82.3725) (width 0.2) (layer "F.Cu") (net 6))
 (via (at 151.17 82.37) (size 0.6) (drill 0.3) (layers "F.Cu" "B.Cu") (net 6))
 (via (at 153.47 104.44) (size 0.6) (drill 0.3) (layers "F.Cu" "B.Cu") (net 6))
 (via (at 158.75 94.705) (size 0.6) (drill 0.3) (layers "F.Cu" "B.Cu") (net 6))
 (segment (start 158.75 94.705) (end 158.75 102.88) (width 0.2) (layer "B.Cu") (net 6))
 (segment (start 157.19 104.44) (end 153.47 104.44) (width 0.2) (layer "B.Cu") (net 6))
 (segment (start 158.75 102.88) (end 157.19 104.44) (width 0.2) (layer "B.Cu") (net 6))
 (segment (start 158.75 94.705) (end 158.75 82.37) (width 0.2) (layer "B.Cu") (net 6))
 (segment (start 158.75 82.37) (end 151.17 82.37) (width 0.2) (layer "B.Cu") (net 6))
 (segment (start 155.3925 86.03) (end 161.17 86.03) (width 0.2) (layer "F.Cu") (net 8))
 (segment (start 161.17 86.03) (end 163.19 88.05) (width 0.2) (layer "F.Cu") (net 8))
 (segment (start 150.965 93.435) (end 148.565 93.435) (width 0.2) (layer "F.Cu") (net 14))
 (segment (start 139.73 94.26) (end 132.15 94.26) (width 0.2) (layer "F.Cu") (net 14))
 (segment (start 148.565 93.435) (end 147.77 94.23) (width 0.2) (layer "F.Cu") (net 14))
 (segment (start 132.15 94.26) (end 130.01 92.12) (width 0.2) (layer "F.Cu") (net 14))
 (via (at 147.77 94.23) (size 0.6) (drill 0.3) (layers "F.Cu" "B.Cu") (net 14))
 (via (at 139.73 94.26) (size 0.6) (drill 0.3) (layers "F.Cu" "B.Cu") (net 14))
 (segment (start 147.77 94.23) (end 139.76 94.23) (width 0.2) (layer "B.Cu") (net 14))
 (segment (start 139.76 94.23) (end 139.73 94.26) (width 0.2) (layer "B.Cu") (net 14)))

